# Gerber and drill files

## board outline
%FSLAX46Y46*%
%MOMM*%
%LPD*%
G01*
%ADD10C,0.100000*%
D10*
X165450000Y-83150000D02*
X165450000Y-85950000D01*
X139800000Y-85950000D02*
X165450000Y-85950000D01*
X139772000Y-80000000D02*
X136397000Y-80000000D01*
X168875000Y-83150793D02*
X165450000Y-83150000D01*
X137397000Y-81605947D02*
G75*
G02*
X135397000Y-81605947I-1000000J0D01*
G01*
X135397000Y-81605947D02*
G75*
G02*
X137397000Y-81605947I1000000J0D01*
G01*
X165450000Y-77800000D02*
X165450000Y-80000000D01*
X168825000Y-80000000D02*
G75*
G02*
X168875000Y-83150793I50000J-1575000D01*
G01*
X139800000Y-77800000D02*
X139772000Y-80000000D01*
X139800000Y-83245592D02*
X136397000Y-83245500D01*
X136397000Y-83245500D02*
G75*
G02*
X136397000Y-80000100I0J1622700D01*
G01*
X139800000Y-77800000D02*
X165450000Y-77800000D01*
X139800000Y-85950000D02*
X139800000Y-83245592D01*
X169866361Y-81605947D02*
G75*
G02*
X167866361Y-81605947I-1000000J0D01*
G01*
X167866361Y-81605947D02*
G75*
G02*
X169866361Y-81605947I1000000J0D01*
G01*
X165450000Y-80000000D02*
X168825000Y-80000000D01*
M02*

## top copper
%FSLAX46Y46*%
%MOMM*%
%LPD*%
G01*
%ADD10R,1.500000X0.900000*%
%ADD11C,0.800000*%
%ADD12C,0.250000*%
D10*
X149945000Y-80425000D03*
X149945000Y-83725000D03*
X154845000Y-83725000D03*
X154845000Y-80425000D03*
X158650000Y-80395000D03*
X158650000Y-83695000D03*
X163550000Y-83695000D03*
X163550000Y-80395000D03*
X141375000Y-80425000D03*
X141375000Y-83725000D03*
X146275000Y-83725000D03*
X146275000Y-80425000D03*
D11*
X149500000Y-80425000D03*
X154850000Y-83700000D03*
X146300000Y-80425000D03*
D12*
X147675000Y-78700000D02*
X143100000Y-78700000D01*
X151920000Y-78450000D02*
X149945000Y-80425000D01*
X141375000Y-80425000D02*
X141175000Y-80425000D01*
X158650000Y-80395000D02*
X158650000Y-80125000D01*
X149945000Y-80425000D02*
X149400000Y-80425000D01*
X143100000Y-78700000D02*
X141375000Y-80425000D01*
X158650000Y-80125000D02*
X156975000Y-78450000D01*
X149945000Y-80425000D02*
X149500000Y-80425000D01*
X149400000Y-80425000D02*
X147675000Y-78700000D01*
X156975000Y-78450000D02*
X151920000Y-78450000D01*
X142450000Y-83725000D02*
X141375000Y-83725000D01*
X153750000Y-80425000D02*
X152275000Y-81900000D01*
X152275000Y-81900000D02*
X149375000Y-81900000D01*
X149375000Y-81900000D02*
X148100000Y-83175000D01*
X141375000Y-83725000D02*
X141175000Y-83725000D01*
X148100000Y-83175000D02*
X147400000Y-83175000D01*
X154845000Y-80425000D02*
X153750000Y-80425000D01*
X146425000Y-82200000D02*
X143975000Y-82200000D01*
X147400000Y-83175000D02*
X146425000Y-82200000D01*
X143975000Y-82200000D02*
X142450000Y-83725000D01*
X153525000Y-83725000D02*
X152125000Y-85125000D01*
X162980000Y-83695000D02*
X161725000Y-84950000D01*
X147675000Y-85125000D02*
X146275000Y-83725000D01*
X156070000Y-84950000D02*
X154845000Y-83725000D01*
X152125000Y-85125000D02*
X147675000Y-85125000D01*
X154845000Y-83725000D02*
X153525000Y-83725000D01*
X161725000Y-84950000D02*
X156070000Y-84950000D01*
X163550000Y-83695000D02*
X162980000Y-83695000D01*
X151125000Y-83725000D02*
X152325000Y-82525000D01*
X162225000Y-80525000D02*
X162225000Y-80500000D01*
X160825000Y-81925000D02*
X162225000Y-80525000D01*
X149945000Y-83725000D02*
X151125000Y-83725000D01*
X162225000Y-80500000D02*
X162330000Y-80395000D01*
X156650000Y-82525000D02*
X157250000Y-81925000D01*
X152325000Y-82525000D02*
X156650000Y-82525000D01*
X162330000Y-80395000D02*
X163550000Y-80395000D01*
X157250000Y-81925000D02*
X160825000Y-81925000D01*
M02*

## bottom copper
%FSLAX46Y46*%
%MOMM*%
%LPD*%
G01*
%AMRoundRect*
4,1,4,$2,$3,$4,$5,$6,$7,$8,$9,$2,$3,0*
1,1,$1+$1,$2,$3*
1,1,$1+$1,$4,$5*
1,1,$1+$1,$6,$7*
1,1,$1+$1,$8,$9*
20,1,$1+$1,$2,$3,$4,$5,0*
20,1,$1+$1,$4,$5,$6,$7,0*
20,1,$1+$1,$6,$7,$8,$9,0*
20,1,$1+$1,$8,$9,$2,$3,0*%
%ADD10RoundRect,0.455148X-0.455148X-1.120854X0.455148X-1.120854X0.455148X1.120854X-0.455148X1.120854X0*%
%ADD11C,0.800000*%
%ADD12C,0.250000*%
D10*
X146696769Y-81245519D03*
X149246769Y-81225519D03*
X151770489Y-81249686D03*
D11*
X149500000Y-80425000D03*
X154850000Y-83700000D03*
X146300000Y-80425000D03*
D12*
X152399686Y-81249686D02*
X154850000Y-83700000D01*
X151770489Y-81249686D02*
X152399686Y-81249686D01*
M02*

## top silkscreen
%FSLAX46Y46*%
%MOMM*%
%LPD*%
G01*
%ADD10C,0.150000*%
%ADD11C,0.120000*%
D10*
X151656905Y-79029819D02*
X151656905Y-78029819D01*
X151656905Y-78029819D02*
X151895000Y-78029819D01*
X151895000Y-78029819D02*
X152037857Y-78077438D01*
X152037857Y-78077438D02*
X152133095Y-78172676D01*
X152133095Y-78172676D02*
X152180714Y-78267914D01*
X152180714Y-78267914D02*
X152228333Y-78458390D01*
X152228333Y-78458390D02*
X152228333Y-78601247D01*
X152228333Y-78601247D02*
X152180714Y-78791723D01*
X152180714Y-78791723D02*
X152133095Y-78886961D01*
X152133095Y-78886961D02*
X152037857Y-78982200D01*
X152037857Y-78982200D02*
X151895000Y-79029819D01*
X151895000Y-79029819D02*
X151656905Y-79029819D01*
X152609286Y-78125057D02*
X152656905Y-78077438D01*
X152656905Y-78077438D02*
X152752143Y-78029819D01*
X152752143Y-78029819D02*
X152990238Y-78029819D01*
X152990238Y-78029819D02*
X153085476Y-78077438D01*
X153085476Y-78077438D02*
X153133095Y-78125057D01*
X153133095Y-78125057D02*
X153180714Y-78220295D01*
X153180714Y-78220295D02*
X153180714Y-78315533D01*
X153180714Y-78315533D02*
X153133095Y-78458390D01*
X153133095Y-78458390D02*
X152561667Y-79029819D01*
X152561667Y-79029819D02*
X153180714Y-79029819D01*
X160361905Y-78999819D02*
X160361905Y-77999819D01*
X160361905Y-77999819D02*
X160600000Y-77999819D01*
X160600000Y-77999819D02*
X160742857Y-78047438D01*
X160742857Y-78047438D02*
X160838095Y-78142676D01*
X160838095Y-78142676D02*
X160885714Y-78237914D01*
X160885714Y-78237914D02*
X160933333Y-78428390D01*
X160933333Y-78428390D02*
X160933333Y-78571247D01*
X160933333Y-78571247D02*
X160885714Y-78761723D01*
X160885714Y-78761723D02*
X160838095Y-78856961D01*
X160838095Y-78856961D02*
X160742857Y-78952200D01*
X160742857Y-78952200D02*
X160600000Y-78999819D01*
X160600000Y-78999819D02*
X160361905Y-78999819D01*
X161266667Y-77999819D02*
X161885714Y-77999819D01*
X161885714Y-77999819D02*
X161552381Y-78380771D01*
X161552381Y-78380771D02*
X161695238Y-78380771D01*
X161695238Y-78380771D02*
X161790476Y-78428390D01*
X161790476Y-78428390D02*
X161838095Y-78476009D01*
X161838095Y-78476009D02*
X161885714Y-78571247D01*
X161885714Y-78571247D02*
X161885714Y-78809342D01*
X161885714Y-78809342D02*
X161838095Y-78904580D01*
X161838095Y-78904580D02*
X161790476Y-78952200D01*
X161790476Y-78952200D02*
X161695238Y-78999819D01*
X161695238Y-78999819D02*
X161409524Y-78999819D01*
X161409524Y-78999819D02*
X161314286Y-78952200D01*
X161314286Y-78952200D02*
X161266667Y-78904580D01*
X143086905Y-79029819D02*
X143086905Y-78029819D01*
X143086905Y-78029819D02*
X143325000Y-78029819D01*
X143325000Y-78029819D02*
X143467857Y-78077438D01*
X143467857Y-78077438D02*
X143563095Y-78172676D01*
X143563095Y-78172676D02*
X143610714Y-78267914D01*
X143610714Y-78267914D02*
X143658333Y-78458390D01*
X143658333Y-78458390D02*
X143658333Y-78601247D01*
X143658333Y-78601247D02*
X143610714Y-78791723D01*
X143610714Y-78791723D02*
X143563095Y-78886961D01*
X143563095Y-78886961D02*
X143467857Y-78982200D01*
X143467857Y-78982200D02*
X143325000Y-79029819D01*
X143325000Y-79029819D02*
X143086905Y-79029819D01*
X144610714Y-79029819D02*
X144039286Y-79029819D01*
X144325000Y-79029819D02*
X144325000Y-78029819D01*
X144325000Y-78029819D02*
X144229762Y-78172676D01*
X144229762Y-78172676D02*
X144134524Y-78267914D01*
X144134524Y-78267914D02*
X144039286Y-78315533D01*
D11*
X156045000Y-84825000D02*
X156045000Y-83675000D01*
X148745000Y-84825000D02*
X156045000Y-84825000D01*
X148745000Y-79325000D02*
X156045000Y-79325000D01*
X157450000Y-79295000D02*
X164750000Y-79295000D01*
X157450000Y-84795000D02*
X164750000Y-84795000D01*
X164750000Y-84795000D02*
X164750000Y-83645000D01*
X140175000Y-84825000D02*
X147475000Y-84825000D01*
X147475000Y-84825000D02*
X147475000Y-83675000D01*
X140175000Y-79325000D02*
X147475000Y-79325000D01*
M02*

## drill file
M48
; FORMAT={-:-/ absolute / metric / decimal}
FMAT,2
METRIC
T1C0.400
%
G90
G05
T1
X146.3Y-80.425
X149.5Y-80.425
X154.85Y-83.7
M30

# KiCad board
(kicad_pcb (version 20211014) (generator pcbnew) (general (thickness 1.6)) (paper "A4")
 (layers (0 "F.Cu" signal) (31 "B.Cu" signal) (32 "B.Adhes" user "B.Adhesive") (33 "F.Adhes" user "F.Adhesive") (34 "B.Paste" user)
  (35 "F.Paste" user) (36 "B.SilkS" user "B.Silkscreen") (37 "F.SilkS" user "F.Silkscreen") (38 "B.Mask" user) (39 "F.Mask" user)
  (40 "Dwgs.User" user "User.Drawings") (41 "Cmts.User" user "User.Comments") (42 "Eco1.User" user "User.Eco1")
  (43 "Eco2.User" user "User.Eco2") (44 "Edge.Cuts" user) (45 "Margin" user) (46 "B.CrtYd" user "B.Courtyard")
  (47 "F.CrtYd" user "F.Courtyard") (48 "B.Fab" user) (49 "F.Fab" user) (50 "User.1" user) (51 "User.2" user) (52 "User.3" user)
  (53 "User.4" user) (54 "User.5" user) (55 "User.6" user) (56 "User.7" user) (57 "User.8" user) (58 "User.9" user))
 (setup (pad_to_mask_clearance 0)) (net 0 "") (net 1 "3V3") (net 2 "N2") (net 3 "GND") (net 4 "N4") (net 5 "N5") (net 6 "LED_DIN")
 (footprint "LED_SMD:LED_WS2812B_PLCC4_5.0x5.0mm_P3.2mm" (layer "F.Cu") (at 152.395 82.075)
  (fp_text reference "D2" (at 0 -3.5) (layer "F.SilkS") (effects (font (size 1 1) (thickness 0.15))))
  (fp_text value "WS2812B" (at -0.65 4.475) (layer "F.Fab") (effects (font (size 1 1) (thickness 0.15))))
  (fp_line (start 3.65 2.75) (end 3.65 1.6) (layer "F.SilkS") (width 0.12))
  (fp_line (start -3.65 2.75) (end 3.65 2.75) (layer "F.SilkS") (width 0.12))
  (fp_line (start -3.65 -2.75) (end 3.65 -2.75) (layer "F.SilkS") (width 0.12))
  (pad "1" smd rect (at -2.45 -1.65) (size 1.5 0.9) (layers "F.Cu" "F.Paste" "F.Mask") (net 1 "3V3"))
  (pad "2" smd rect (at -2.45 1.65) (size 1.5 0.9) (layers "F.Cu" "F.Paste" "F.Mask") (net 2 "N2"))
  (pad "3" smd rect (at 2.45 1.65) (size 1.5 0.9) (layers "F.Cu" "F.Paste" "F.Mask") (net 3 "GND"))
  (pad "4" smd rect (at 2.45 -1.65) (size 1.5 0.9) (layers "F.Cu" "F.Paste" "F.Mask") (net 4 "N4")))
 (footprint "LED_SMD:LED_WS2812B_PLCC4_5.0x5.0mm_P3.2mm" (layer "F.Cu") (at 161.1 82.045)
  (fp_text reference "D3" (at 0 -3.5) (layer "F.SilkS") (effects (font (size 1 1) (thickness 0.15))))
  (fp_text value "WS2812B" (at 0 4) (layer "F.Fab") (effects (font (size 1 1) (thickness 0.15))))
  (fp_line (start -3.65 -2.75) (end 3.65 -2.75) (layer "F.SilkS") (width 0.12))
  (fp_line (start -3.65 2.75) (end 3.65 2.75) (layer "F.SilkS") (width 0.12))
  (fp_line (start 3.65 2.75) (end 3.65 1.6) (layer "F.SilkS") (width 0.12))
  (pad "1" smd rect (at -2.45 -1.65) (size 1.5 0.9) (layers "F.Cu" "F.Paste" "F.Mask") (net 1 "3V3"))
  (pad "2" smd rect (at -2.45 1.65) (size 1.5 0.9) (layers "F.Cu" "F.Paste" "F.Mask") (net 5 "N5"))
  (pad "3" smd rect (at 2.45 1.65) (size 1.5 0.9) (layers "F.Cu" "F.Paste" "F.Mask") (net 3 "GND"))
  (pad "4" smd rect (at 2.45 -1.65) (size 1.5 0.9) (layers "F.Cu" "F.Paste" "F.Mask") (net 2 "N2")))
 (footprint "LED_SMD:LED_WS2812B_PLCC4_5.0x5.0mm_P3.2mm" (layer "F.Cu") (at 143.825 82.075)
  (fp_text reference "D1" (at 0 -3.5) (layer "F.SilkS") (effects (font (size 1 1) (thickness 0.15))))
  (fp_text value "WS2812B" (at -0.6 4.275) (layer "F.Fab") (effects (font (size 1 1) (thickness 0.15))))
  (fp_line (start -3.65 2.75) (end 3.65 2.75) (layer "F.SilkS") (width 0.12))
  (fp_line (start 3.65 2.75) (end 3.65 1.6) (layer "F.SilkS") (width 0.12))
  (fp_line (start -3.65 -2.75) (end 3.65 -2.75) (layer "F.SilkS") (width 0.12))
  (pad "1" smd rect (at -2.45 -1.65) (size 1.5 0.9) (layers "F.Cu" "F.Paste" "F.Mask") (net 1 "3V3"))
  (pad "2" smd rect (at -2.45 1.65) (size 1.5 0.9) (layers "F.Cu" "F.Paste" "F.Mask") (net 4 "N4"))
  (pad "3" smd rect (at 2.45 1.65) (size 1.5 0.9) (layers "F.Cu" "F.Paste" "F.Mask") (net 3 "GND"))
  (pad "4" smd rect (at 2.45 -1.65) (size 1.5 0.9) (layers "F.Cu" "F.Paste" "F.Mask") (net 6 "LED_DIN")))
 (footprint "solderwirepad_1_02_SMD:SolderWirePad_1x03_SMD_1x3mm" (layer "B.Cu") (at 146.72 81.214167)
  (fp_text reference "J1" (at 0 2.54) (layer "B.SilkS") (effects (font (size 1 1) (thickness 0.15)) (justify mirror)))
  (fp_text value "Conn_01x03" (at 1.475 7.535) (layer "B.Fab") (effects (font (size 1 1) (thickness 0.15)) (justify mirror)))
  (pad "1" smd roundrect (at -0.023231 0.031352) (size 1.820592 3.152005) (layers "B.Cu" "B.Paste" "B.Mask") (roundrect_rratio 0.25)
   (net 6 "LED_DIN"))
  (pad "2" smd roundrect (at 2.526769 0.011352) (size 1.820592 3.152005) (layers "B.Cu" "B.Paste" "B.Mask") (roundrect_rratio 0.25)
   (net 1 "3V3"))
  (pad "3" smd roundrect (at 5.050489 0.035519) (size 1.820592 3.152005) (layers "B.Cu" "B.Paste" "B.Mask") (roundrect_rratio 0.25)
   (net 3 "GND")))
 (gr_line (start 165.45 83.15) (end 165.45 85.95) (layer "Edge.Cuts") (width 0.1))
 (gr_line (start 139.8 85.95) (end 165.45 85.95) (layer "Edge.Cuts") (width 0.1))
 (gr_line (start 139.772 80) (end 136.397 80) (layer "Edge.Cuts") (width 0.1))
 (gr_line (start 168.875 83.150793) (end 165.45 83.15) (layer "Edge.Cuts") (width 0.1))
 (gr_circle (center 136.397 81.605947) (end 137.397 81.605947) (layer "Edge.Cuts") (width 0.1) (fill none))
 (gr_line (start 165.45 77.8) (end 165.45 80) (layer "Edge.Cuts") (width 0.1))
 (gr_arc (start 168.825 80) (mid 170.450595 81.549997) (end 168.875 83.150793) (layer "Edge.Cuts") (width 0.1))
 (gr_line (start 139.8 77.8) (end 139.772 80) (layer "Edge.Cuts") (width 0.1))
 (gr_line (start 139.8 83.245592) (end 136.397 83.2455) (layer "Edge.Cuts") (width 0.1))
 (gr_arc (start 136.397 83.2455) (mid 134.77425 81.62275) (end 136.397 80) (layer "Edge.Cuts") (width 0.1))
 (gr_line (start 139.8 77.8) (end 165.45 77.8) (layer "Edge.Cuts") (width 0.1))
 (gr_line (start 139.8 85.95) (end 139.8 83.245592) (layer "Edge.Cuts") (width 0.1))
 (gr_circle (center 168.866361 81.605947) (end 169.866361 81.605947) (layer "Edge.Cuts") (width 0.1) (fill none))
 (gr_line (start 165.45 80) (end 168.825 80) (layer "Edge.Cuts") (width 0.1))
 (segment (start 147.675 78.7) (end 143.1 78.7) (width 0.25) (layer "F.Cu") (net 1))
 (segment (start 151.92 78.45) (end 149.945 80.425) (width 0.25) (layer "F.Cu") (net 1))
 (segment (start 141.375 80.425) (end 141.175 80.425) (width 0.25) (layer "F.Cu") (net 1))
 (segment (start 158.65 80.395) (end 158.65 80.125) (width 0.25) (layer "F.Cu") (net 1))
 (segment (start 149.945 80.425) (end 149.4 80.425) (width 0.25) (layer "F.Cu") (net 1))
 (segment (start 143.1 78.7) (end 141.375 80.425) (width 0.25) (layer "F.Cu") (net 1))
 (segment (start 158.65 80.125) (end 156.975 78.45) (width 0.25) (layer "F.Cu") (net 1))
 (segment (start 149.945 80.425) (end 149.5 80.425) (width 0.25) (layer "F.Cu") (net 1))
 (segment (start 149.4 80.425) (end 147.675 78.7) (width 0.25) (layer "F.Cu") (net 1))
 (segment (start 156.975 78.45) (end 151.92 78.45) (width 0.25) (layer "F.Cu") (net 1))
 (via (at 149.5 80.425) (size 0.8) (drill 0.4) (layers "F.Cu" "B.Cu") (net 1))
 (segment (start 142.45 83.725) (end 141.375 83.725) (width 0.25) (layer "F.Cu") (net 4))
 (segment (start 153.75 80.425) (end 152.275 81.9) (width 0.25) (layer "F.Cu") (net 4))
 (segment (start 152.275 81.9) (end 149.375 81.9) (width 0.25) (layer "F.Cu") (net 4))
 (segment (start 149.375 81.9) (end 148.1 83.175) (width 0.25) (layer "F.Cu") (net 4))
 (segment (start 141.375 83.725) (end 141.175 83.725) (width 0.25) (layer "F.Cu") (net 4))
 (segment (start 148.1 83.175) (end 147.4 83.175) (width 0.25) (layer "F.Cu") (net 4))
 (segment (start 154.845 80.425) (end 153.75 80.425) (width 0.25) (layer "F.Cu") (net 4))
 (segment (start 146.425 82.2) (end 143.975 82.2) (width 0.25) (layer "F.Cu") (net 4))
 (segment (start 147.4 83.175) (end 146.425 82.2) (width 0.25) (layer "F.Cu") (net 4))
 (segment (start 143.975 82.2) (end 142.45 83.725) (width 0.25) (layer "F.Cu") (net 4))
 (segment (start 153.525 83.725) (end 152.125 85.125) (width 0.25) (layer "F.Cu") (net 3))
 (segment (start 162.98 83.695) (end 161.725 84.95) (width 0.25) (layer "F.Cu") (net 3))
 (segment (start 147.675 85.125) (end 146.275 83.725) (width 0.25) (layer "F.Cu") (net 3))
 (segment (start 156.07 84.95) (end 154.845 83.725) (width 0.25) (layer "F.Cu") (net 3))
 (segment (start 152.125 85.125) (end 147.675 85.125) (width 0.25) (layer "F.Cu") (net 3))
 (segment (start 154.845 83.725) (end 153.525 83.725) (width 0.25) (layer "F.Cu") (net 3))
 (segment (start 161.725 84.95) (end 156.07 84.95) (width 0.25) (layer "F.Cu") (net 3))
 (segment (start 163.55 83.695) (end 162.98 83.695) (width 0.25) (layer "F.Cu") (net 3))
 (via (at 154.85 83.7) (size 0.8) (drill 0.4) (layers "F.Cu" "B.Cu") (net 3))
 (segment (start 152.399686 81.249686) (end 154.85 83.7) (width 0.25) (layer "B.Cu") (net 3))
 (segment (start 151.770489 81.249686) (end 152.399686 81.249686) (width 0.25) (layer "B.Cu") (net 3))
 (via (at 146.3 80.425) (size 0.8) (drill 0.4) (layers "F.Cu" "B.Cu") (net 6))
 (segment (start 151.125 83.725) (end 152.325 82.525) (width 0.25) (layer "F.Cu") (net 2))
 (segment (start 162.225 80.525) (end 162.225 80.5) (width 0.25) (layer "F.Cu") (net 2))
 (segment (start 160.825 81.925) (end 162.225 80.525) (width 0.25) (layer "F.Cu") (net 2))
 (segment (start 149.945 83.725) (end 151.125 83.725) (width 0.25) (layer "F.Cu") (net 2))
 (segment (start 162.225 80.5) (end 162.33 80.395) (width 0.25) (layer "F.Cu") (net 2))
 (segment (start 156.65 82.525) (end 157.25 81.925) (width 0.25) (layer "F.Cu") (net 2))
 (segment (start 152.325 82.525) (end 156.65 82.525) (width 0.25) (layer "F.Cu") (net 2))
 (segment (start 162.33 80.395) (end 163.55 80.395) (width 0.25) (layer "F.Cu") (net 2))
 (segment (start 157.25 81.925) (end 160.825 81.925) (width 0.25) (layer "F.Cu") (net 2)))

